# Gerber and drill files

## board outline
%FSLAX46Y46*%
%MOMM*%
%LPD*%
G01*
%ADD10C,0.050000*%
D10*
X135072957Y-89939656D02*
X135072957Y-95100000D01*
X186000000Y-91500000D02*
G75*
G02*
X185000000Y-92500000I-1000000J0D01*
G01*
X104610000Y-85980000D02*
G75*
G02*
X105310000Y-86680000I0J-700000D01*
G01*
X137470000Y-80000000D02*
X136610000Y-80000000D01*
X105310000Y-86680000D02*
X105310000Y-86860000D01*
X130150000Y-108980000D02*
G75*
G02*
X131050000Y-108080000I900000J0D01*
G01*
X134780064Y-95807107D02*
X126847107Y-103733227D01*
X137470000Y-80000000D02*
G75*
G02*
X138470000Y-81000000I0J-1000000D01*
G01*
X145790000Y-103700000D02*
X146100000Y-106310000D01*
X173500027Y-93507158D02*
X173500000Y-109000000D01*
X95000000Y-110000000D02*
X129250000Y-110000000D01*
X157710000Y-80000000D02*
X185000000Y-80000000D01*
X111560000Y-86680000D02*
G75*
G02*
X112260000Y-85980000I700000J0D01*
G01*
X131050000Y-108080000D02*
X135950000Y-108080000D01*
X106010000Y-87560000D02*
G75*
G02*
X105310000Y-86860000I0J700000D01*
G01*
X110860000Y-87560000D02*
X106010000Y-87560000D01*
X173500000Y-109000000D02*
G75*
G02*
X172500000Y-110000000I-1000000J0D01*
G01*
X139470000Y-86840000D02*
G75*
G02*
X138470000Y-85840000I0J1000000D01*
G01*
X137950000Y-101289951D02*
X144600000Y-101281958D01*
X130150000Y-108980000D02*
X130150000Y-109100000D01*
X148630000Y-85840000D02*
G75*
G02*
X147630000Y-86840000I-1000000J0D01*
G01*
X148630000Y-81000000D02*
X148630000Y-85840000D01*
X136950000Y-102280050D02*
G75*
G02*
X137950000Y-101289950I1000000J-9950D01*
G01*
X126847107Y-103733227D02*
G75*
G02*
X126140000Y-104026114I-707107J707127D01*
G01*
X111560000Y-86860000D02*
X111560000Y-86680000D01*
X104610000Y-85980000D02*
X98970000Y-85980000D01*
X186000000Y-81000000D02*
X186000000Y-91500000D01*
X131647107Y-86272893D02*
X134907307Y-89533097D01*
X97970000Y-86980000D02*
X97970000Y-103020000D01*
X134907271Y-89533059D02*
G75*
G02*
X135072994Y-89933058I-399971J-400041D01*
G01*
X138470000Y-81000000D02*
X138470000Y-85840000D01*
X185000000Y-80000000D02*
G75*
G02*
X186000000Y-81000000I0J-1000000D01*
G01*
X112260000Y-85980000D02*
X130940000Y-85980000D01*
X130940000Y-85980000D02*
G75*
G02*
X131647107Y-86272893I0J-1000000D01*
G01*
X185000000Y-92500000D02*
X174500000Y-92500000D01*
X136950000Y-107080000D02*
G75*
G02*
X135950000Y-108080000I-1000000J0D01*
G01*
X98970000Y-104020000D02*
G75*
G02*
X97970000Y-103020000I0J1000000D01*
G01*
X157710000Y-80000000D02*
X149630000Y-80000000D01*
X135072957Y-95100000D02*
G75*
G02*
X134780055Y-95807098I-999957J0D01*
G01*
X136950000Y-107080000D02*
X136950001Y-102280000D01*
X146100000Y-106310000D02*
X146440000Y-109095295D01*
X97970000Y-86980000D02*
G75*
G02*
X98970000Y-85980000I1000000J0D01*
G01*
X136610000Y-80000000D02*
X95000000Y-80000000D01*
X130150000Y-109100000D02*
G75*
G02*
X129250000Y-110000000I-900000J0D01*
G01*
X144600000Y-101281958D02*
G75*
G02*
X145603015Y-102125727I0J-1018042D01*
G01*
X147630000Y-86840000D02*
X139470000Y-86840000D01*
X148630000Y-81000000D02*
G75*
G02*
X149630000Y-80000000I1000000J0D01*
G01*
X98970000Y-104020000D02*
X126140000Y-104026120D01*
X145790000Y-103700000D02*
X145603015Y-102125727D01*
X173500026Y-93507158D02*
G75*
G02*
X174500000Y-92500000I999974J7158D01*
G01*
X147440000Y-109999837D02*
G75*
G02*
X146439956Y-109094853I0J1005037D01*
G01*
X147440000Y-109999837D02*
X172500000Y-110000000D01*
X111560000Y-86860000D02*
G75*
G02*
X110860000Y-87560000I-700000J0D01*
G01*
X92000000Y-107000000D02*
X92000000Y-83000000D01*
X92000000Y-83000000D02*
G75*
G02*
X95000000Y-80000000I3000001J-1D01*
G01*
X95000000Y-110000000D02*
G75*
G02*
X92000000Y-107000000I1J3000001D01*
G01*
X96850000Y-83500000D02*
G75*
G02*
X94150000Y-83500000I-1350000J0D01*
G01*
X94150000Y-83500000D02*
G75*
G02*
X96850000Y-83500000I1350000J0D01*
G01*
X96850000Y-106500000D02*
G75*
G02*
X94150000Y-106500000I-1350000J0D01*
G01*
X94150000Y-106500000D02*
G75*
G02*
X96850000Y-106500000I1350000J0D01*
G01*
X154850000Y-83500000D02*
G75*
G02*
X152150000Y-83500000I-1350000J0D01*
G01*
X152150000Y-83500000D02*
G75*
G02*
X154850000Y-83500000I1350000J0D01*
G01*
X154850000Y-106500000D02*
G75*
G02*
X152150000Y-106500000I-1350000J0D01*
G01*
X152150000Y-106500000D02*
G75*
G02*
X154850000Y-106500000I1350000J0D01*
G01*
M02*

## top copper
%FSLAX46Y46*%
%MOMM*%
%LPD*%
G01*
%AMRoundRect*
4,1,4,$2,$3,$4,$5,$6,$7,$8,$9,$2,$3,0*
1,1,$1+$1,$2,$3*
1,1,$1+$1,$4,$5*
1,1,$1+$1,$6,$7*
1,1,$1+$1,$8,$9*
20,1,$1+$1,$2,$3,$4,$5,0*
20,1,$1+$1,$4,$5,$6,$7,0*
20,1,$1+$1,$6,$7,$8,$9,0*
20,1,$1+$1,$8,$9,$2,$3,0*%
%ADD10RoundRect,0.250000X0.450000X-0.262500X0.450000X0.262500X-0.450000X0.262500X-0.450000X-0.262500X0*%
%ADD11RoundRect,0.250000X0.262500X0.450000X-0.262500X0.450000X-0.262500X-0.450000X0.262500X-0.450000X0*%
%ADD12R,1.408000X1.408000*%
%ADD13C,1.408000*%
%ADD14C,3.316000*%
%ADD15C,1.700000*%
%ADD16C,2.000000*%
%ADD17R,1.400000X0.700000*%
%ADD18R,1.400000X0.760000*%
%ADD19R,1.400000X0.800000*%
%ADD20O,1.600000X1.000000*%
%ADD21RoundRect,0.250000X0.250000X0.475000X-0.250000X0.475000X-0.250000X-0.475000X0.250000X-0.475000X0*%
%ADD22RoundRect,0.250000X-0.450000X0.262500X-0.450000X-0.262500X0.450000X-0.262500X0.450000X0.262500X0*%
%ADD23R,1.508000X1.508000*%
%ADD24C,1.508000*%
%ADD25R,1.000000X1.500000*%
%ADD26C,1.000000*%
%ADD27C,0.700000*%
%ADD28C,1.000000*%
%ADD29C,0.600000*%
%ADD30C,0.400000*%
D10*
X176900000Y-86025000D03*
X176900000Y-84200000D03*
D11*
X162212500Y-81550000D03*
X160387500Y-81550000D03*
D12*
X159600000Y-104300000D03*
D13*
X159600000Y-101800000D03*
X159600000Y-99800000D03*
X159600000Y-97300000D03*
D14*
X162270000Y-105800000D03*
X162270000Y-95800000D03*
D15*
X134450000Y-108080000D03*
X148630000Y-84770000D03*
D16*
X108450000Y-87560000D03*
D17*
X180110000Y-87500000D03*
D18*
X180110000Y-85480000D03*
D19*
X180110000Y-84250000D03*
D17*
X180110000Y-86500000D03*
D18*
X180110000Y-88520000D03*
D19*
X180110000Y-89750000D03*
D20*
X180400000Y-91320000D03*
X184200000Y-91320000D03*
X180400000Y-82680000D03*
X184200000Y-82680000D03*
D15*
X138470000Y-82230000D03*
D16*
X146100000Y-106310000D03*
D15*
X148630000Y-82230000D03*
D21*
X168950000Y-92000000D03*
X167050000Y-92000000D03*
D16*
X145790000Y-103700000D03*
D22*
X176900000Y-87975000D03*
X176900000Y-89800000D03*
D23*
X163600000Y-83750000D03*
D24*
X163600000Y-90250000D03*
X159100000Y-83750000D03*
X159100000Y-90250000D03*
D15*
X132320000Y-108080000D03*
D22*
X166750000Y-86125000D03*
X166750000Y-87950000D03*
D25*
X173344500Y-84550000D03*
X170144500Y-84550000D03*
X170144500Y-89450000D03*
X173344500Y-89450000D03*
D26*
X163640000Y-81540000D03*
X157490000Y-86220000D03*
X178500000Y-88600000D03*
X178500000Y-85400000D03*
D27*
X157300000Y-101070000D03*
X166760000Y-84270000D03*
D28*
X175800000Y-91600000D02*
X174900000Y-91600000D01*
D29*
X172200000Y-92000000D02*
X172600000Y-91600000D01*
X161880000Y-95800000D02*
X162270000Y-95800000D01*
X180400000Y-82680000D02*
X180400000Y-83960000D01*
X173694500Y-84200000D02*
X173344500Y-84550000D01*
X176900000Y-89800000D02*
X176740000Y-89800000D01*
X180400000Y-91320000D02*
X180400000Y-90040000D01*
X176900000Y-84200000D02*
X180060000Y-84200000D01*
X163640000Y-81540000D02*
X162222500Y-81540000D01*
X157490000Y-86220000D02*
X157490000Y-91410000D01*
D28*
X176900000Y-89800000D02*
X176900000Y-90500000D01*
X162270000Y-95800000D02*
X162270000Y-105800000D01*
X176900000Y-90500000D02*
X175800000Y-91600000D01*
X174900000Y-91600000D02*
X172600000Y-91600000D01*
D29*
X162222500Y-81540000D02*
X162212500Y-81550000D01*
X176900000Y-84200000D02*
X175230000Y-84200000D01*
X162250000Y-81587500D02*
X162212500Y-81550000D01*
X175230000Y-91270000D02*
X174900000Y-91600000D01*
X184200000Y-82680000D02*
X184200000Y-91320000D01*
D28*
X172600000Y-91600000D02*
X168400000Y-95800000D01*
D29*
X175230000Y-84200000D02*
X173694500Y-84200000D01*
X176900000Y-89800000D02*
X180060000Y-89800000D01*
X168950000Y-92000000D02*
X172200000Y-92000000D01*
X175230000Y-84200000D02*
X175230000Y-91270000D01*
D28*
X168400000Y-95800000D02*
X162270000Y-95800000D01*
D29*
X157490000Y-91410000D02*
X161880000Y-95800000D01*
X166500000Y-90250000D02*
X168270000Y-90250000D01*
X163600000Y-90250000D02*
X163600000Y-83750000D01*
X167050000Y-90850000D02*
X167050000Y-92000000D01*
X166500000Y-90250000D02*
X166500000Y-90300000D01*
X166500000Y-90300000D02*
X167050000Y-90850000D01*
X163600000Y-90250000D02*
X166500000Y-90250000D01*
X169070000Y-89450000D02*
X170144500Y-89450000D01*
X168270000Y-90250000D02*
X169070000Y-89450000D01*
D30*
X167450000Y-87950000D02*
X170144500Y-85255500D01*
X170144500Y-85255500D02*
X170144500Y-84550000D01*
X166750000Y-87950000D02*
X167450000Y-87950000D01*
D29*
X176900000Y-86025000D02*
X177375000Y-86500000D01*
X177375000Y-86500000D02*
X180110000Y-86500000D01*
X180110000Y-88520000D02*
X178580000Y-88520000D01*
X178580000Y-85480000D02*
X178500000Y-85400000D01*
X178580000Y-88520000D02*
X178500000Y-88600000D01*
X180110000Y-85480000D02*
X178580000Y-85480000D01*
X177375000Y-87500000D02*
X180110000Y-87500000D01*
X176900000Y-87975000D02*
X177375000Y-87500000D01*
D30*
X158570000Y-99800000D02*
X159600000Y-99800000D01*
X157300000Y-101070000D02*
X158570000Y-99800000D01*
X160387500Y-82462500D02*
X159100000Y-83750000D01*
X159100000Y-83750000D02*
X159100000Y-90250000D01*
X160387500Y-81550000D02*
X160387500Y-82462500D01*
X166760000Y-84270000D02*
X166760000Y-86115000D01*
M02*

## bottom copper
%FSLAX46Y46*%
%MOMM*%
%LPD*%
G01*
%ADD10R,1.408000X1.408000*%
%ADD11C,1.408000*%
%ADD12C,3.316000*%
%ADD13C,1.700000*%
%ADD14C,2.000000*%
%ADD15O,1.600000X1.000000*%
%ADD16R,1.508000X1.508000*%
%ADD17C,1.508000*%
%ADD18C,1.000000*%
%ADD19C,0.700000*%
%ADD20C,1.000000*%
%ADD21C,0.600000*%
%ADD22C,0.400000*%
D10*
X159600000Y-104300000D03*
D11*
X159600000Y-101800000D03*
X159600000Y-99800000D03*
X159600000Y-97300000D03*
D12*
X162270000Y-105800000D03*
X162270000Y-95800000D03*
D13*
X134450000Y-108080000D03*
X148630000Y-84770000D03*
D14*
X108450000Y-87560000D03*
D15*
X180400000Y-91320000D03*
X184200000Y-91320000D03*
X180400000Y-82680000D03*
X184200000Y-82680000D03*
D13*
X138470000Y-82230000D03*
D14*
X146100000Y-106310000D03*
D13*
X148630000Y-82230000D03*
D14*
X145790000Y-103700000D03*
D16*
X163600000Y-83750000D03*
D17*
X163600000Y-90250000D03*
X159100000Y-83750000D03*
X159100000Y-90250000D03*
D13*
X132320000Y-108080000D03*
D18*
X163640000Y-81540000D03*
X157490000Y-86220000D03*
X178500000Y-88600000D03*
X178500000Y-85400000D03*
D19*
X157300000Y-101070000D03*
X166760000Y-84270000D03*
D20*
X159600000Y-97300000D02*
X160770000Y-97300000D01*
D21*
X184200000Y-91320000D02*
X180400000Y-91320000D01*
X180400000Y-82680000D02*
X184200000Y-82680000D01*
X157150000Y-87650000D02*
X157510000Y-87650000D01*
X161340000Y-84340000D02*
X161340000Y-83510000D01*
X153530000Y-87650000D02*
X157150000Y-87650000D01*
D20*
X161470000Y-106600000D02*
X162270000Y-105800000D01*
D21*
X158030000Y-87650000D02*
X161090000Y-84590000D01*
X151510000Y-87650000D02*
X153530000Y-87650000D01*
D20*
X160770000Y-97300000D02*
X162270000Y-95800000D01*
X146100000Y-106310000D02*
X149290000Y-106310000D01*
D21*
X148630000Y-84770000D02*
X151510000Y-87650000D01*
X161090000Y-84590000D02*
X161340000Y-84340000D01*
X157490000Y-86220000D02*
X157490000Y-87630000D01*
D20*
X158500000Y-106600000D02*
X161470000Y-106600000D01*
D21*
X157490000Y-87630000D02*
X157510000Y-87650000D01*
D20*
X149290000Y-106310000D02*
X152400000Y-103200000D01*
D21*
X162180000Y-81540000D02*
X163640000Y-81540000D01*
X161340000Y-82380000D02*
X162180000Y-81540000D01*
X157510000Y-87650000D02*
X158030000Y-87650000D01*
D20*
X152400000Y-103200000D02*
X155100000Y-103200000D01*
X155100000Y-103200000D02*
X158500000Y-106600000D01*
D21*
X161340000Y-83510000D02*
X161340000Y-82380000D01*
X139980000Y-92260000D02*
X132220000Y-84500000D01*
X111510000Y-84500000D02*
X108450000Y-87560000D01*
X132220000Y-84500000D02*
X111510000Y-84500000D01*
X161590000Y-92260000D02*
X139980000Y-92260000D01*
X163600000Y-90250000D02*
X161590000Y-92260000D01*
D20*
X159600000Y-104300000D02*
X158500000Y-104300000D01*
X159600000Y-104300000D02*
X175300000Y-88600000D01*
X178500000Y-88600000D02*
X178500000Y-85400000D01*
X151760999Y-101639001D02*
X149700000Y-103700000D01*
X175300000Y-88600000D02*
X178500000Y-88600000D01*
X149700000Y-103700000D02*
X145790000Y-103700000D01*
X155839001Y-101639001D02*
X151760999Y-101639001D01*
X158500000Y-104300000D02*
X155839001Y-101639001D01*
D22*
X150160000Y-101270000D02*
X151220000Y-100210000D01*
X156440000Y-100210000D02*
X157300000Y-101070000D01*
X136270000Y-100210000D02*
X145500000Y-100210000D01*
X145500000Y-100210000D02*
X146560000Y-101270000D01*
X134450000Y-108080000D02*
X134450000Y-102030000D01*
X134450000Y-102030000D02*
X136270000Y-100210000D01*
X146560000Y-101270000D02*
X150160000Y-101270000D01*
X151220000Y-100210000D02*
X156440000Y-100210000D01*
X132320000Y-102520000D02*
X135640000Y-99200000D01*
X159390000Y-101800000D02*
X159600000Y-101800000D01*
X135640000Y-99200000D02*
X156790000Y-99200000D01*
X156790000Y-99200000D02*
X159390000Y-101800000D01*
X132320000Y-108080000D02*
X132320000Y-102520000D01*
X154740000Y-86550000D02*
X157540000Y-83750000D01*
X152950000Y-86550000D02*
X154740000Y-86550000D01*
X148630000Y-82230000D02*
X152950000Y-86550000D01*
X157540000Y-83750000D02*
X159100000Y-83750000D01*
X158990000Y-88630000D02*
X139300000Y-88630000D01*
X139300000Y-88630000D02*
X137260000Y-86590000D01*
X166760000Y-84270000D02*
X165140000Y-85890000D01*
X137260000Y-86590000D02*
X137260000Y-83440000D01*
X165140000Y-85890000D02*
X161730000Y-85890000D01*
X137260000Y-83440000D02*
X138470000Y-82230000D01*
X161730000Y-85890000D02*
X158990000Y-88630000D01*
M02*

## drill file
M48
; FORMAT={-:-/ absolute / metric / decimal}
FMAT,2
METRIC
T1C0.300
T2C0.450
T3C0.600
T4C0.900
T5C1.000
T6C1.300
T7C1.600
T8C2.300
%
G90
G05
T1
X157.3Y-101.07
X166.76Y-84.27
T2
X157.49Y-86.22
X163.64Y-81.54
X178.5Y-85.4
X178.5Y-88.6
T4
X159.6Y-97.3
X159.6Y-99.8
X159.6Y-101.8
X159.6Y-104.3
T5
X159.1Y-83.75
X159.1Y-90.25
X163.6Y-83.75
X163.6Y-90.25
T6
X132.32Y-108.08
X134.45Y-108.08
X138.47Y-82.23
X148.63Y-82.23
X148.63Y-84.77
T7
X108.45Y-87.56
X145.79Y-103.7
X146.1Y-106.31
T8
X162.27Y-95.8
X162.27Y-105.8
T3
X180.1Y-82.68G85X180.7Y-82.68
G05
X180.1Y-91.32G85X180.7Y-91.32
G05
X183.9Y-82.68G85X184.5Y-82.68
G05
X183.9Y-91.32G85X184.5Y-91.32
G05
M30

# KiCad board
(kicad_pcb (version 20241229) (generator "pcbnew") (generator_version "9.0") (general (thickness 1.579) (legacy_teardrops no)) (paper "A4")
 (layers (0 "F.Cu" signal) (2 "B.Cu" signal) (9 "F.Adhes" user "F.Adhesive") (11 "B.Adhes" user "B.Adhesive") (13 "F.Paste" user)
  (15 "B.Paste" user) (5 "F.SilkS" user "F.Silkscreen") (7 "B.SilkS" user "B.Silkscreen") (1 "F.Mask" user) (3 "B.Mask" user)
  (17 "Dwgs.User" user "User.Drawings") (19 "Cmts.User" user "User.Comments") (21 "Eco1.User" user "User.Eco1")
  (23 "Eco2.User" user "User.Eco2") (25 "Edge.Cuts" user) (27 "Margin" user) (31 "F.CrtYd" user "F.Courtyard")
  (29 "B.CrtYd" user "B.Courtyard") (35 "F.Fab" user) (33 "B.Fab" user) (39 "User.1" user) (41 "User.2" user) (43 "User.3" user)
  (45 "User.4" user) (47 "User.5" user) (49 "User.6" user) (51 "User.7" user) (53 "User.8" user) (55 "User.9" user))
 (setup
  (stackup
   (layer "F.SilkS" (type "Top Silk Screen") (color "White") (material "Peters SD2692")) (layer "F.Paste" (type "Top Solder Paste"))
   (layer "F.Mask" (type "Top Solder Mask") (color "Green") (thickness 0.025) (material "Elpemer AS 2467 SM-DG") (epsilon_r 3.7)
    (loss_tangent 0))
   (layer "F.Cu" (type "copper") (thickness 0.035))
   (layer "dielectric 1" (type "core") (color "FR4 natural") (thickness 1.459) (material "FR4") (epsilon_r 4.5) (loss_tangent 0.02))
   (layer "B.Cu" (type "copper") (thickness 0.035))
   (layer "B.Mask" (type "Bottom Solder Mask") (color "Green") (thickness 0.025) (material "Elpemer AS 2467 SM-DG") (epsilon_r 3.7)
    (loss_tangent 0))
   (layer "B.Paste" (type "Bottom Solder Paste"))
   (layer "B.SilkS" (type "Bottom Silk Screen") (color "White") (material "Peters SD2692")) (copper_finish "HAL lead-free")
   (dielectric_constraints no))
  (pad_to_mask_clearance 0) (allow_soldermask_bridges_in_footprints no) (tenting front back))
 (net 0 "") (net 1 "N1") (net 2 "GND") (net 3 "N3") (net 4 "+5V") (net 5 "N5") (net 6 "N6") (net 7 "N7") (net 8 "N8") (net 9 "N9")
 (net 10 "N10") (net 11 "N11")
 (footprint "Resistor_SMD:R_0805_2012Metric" (layer "F.Cu") (at 176.9 85.1125 90)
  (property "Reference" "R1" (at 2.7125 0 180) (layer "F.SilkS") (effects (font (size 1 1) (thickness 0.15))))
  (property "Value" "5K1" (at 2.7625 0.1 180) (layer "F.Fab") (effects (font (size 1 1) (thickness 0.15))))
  (pad "1" smd roundrect (at -0.9125 0 90) (size 1.025 1.4) (layers "F.Cu" "F.Mask" "F.Paste") (roundrect_rratio 0.243902) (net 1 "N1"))
  (pad "2" smd roundrect (at 0.9125 0 90) (size 1.025 1.4) (layers "F.Cu" "F.Mask" "F.Paste") (roundrect_rratio 0.243902) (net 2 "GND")))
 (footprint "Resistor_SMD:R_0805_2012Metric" (layer "F.Cu") (at 161.3 81.55 180)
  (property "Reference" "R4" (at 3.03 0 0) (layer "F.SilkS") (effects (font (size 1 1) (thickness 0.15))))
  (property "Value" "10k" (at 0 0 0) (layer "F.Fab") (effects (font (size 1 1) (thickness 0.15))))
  (pad "1" smd roundrect (at -0.9125 0 180) (size 1.025 1.4) (layers "F.Cu" "F.Mask" "F.Paste") (roundrect_rratio 0.243902) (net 2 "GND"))
  (pad "2" smd roundrect (at 0.9125 0 180) (size 1.025 1.4) (layers "F.Cu" "F.Mask" "F.Paste") (roundrect_rratio 0.243902) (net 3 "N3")))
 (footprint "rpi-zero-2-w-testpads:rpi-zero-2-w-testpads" (layer "F.Cu") (at 157 110)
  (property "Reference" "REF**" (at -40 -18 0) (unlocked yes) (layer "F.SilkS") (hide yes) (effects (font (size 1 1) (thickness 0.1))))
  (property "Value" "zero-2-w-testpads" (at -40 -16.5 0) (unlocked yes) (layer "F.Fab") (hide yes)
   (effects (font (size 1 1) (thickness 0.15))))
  (fp_line (start -65 -3) (end -65 -27) (stroke (width 0.05) (type solid)) (layer "Edge.Cuts"))
  (fp_arc (start -65 -27) (mid -64.12132 -29.12132) (end -62 -30) (stroke (width 0.05) (type solid)) (layer "Edge.Cuts"))
  (fp_arc (start -62 0) (mid -64.12132 -0.87868) (end -65 -3) (stroke (width 0.05) (type solid)) (layer "Edge.Cuts"))
  (fp_circle (center -61.5 -26.5) (end -60.15 -26.5) (stroke (width 0.05) (type solid)) (fill no) (layer "Edge.Cuts"))
  (fp_circle (center -61.5 -3.5) (end -60.15 -3.5) (stroke (width 0.05) (type solid)) (fill no) (layer "Edge.Cuts"))
  (fp_circle (center -3.5 -26.5) (end -2.15 -26.5) (stroke (width 0.05) (type solid)) (fill no) (layer "Edge.Cuts"))
  (fp_circle (center -3.5 -3.5) (end -2.15 -3.5) (stroke (width 0.05) (type solid)) (fill no) (layer "Edge.Cuts"))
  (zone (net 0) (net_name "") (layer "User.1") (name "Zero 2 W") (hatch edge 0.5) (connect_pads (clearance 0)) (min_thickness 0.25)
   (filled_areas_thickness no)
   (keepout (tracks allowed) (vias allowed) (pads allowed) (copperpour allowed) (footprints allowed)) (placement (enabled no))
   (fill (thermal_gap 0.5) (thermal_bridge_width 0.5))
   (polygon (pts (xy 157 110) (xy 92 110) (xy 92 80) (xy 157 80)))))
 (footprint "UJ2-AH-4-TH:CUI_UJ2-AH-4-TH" (layer "F.Cu") (at 159.6 104.3 90)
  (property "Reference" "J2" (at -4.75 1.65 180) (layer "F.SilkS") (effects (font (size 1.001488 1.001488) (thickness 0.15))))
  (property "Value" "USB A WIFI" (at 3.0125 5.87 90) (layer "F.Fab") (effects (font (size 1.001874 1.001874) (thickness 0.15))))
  (pad "1" thru_hole rect (at 0 0 90) (size 1.408 1.408) (drill 0.9) (layers "*.Cu" "*.Mask") (remove_unused_layers no) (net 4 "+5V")
   (solder_mask_margin 0.102))
  (pad "2" thru_hole circle (at 2.5 0 90) (size 1.408 1.408) (drill 0.9) (layers "*.Cu" "*.Mask") (remove_unused_layers no) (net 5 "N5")
   (solder_mask_margin 0.102))
  (pad "3" thru_hole circle (at 4.5 0 90) (size 1.408 1.408) (drill 0.9) (layers "*.Cu" "*.Mask") (remove_unused_layers no) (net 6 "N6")
   (solder_mask_margin 0.102))
  (pad "4" thru_hole circle (at 7 0 90) (size 1.408 1.408) (drill 0.9) (layers "*.Cu" "*.Mask") (remove_unused_layers no) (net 2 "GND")
   (solder_mask_margin 0.102))
  (pad "SH1" thru_hole circle (at -1.5 2.67 90) (size 3.316 3.316) (drill 2.3) (layers "*.Cu" "*.Mask") (remove_unused_layers no)
   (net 2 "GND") (solder_mask_margin 0.102))
  (pad "SH2" thru_hole circle (at 8.5 2.67 90) (size 3.316 3.316) (drill 2.3) (layers "*.Cu" "*.Mask") (remove_unused_layers no)
   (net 2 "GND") (solder_mask_margin 0.102)))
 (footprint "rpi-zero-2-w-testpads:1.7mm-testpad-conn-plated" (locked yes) (layer "F.Cu") (at 134.45 108.08)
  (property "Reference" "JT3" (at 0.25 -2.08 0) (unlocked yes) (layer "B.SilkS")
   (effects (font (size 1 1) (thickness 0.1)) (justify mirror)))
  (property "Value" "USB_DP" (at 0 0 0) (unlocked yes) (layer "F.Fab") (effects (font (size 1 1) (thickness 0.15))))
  (pad "1" thru_hole circle (at 0 0) (size 1.7 1.7) (drill 1.3) (layers "*.Cu" "*.Mask") (remove_unused_layers no) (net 6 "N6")))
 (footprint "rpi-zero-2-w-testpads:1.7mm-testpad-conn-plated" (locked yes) (layer "F.Cu") (at 148.63 84.77)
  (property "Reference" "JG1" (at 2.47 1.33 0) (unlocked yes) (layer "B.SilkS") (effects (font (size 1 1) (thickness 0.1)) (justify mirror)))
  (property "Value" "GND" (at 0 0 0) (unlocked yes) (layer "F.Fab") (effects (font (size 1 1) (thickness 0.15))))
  (pad "1" thru_hole circle (at 0 0) (size 1.7 1.7) (drill 1.3) (layers "*.Cu" "*.Mask") (remove_unused_layers no) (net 2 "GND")))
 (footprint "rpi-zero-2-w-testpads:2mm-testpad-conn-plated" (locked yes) (layer "F.Cu") (at 108.45 87.56)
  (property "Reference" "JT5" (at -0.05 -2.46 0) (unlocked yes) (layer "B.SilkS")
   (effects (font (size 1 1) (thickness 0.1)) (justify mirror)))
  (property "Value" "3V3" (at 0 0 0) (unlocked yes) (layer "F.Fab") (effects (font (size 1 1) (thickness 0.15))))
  (pad "1" thru_hole circle (at 0 0) (size 2 2) (drill 1.6) (layers "*.Cu" "*.Mask") (remove_unused_layers no) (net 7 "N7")))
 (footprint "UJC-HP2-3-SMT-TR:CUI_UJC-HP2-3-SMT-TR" (layer "F.Cu") (at 184.2 87 90)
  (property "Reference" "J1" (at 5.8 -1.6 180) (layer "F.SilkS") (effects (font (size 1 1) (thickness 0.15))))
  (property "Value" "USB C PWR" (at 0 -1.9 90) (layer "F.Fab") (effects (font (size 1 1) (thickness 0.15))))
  (pad "A5" smd rect (at -0.5 -4.09 90) (size 0.7 1.4) (layers "F.Cu" "F.Mask" "F.Paste") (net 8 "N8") (solder_mask_margin 0.102))
  (pad "A9" smd rect (at 1.52 -4.09 90) (size 0.76 1.4) (layers "F.Cu" "F.Mask" "F.Paste") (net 4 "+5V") (solder_mask_margin 0.102))
  (pad "A12" smd rect (at 2.75 -4.09 90) (size 0.8 1.4) (layers "F.Cu" "F.Mask" "F.Paste") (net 2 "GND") (solder_mask_margin 0.102))
  (pad "B5" smd rect (at 0.5 -4.09 90) (size 0.7 1.4) (layers "F.Cu" "F.Mask" "F.Paste") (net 1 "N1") (solder_mask_margin 0.102))
  (pad "B9" smd rect (at -1.52 -4.09 90) (size 0.76 1.4) (layers "F.Cu" "F.Mask" "F.Paste") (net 4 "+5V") (solder_mask_margin 0.102))
  (pad "B12" smd rect (at -2.75 -4.09 90) (size 0.8 1.4) (layers "F.Cu" "F.Mask" "F.Paste") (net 2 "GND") (solder_mask_margin 0.102))
  (pad "SH1" thru_hole oval (at -4.32 -3.8 90) (size 1 1.6) (drill oval 0.6 1.2) (layers "*.Cu" "*.Mask") (remove_unused_layers no)
   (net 2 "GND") (solder_mask_margin 0.102))
  (pad "SH2" thru_hole oval (at -4.32 0 90) (size 1 1.6) (drill oval 0.6 1.2) (layers "*.Cu" "*.Mask") (remove_unused_layers no)
   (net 2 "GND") (solder_mask_margin 0.102))
  (pad "SH3" thru_hole oval (at 4.32 -3.8 90) (size 1 1.6) (drill oval 0.6 1.2) (layers "*.Cu" "*.Mask") (remove_unused_layers no)
   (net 2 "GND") (solder_mask_margin 0.102))
  (pad "SH4" thru_hole oval (at 4.32 0 90) (size 1 1.6) (drill oval 0.6 1.2) (layers "*.Cu" "*.Mask") (remove_unused_layers no)
   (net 2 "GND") (solder_mask_margin 0.102)))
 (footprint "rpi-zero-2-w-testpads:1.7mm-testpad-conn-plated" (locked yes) (layer "F.Cu") (at 138.47 82.23)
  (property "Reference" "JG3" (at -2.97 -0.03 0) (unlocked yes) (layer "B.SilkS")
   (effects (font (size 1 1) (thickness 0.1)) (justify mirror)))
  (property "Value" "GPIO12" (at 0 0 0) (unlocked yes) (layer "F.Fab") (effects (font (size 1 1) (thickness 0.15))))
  (pad "1" thru_hole circle (at 0 0) (size 1.7 1.7) (drill 1.3) (layers "*.Cu" "*.Mask") (remove_unused_layers no) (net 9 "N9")))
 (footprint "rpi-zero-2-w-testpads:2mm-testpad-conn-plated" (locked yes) (layer "F.Cu") (at 146.1 106.31)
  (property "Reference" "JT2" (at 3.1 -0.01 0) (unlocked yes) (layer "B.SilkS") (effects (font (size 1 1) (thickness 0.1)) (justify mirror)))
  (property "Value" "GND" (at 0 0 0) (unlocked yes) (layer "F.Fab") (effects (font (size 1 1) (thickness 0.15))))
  (pad "1" thru_hole circle (at 0 0) (size 2 2) (drill 1.6) (layers "*.Cu" "*.Mask") (remove_unused_layers no) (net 2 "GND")))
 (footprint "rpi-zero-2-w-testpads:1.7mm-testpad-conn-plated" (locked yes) (layer "F.Cu") (at 148.63 82.23)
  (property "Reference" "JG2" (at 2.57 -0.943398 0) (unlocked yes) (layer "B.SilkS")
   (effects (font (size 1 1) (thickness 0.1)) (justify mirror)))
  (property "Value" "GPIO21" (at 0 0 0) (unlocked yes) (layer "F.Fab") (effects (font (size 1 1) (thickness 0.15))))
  (pad "1" thru_hole circle (at 0 0) (size 1.7 1.7) (drill 1.3) (layers "*.Cu" "*.Mask") (remove_unused_layers no) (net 3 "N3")))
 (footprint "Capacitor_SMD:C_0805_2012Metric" (layer "F.Cu") (at 168 92 180)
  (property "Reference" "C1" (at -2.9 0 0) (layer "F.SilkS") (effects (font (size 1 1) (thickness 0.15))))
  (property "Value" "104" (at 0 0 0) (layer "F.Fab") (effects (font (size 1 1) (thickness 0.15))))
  (pad "1" smd roundrect (at -0.95 0 180) (size 1 1.45) (layers "F.Cu" "F.Mask" "F.Paste") (roundrect_rratio 0.25) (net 2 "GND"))
  (pad "2" smd roundrect (at 0.95 0 180) (size 1 1.45) (layers "F.Cu" "F.Mask" "F.Paste") (roundrect_rratio 0.25) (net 7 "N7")))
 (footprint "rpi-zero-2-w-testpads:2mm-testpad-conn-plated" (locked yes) (layer "F.Cu") (at 145.79 103.7)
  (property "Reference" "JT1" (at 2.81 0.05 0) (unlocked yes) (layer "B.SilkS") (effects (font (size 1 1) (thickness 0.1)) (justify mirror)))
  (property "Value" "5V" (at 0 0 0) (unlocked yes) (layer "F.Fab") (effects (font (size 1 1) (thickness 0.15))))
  (pad "1" thru_hole circle (at 0 0) (size 2 2) (drill 1.6) (layers "*.Cu" "*.Mask") (remove_unused_layers no) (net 4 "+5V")))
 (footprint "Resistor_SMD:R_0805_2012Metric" (layer "F.Cu") (at 176.9 88.8875 -90)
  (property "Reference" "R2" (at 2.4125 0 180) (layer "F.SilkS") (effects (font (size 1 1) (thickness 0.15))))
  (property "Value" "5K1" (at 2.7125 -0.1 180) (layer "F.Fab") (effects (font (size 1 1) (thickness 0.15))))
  (pad "1" smd roundrect (at -0.9125 0 270) (size 1.025 1.4) (layers "F.Cu" "F.Mask" "F.Paste") (roundrect_rratio 0.243902) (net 8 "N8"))
  (pad "2" smd roundrect (at 0.9125 0 270) (size 1.025 1.4) (layers "F.Cu" "F.Mask" "F.Paste") (roundrect_rratio 0.243902) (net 2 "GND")))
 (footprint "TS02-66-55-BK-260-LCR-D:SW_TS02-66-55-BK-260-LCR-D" (layer "F.Cu") (at 161.35 87 -90)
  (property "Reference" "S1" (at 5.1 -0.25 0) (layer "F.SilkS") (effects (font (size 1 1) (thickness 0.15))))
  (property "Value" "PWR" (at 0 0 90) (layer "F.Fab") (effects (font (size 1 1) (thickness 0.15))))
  (pad "1" thru_hole rect (at -3.25 -2.25 270) (size 1.508 1.508) (drill 1) (layers "*.Cu" "*.Mask") (remove_unused_layers no) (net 7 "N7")
   (solder_mask_margin 0.102))
  (pad "2" thru_hole circle (at 3.25 -2.25 270) (size 1.508 1.508) (drill 1) (layers "*.Cu" "*.Mask") (remove_unused_layers no) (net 7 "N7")
   (solder_mask_margin 0.102))
  (pad "3" thru_hole circle (at -3.25 2.25 270) (size 1.508 1.508) (drill 1) (layers "*.Cu" "*.Mask") (remove_unused_layers no) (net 3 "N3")
   (solder_mask_margin 0.102))
  (pad "4" thru_hole circle (at 3.25 2.25 270) (size 1.508 1.508) (drill 1) (layers "*.Cu" "*.Mask") (remove_unused_layers no) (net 3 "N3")
   (solder_mask_margin 0.102)))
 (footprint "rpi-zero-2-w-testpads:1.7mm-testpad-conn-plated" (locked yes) (layer "F.Cu") (at 132.32 108.08)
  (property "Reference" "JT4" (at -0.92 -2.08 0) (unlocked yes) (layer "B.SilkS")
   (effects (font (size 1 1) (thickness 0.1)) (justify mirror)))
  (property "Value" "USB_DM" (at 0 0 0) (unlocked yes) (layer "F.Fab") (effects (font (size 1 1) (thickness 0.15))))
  (pad "1" thru_hole circle (at 0 0) (size 1.7 1.7) (drill 1.3) (layers "*.Cu" "*.Mask") (remove_unused_layers no) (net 5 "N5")))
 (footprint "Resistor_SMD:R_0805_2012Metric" (layer "F.Cu") (at 166.75 87.0375 -90)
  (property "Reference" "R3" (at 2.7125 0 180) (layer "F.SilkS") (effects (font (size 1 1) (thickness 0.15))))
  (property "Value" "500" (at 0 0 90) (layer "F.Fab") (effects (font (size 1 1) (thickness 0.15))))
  (pad "1" smd roundrect (at -0.9125 0 270) (size 1.025 1.4) (layers "F.Cu" "F.Mask" "F.Paste") (roundrect_rratio 0.243902) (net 9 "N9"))
  (pad "2" smd roundrect (at 0.9125 0 270) (size 1.025 1.4) (layers "F.Cu" "F.Mask" "F.Paste") (roundrect_rratio 0.243902) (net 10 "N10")))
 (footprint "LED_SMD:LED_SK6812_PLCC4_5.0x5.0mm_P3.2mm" (layer "F.Cu") (at 171.7445 87 -90)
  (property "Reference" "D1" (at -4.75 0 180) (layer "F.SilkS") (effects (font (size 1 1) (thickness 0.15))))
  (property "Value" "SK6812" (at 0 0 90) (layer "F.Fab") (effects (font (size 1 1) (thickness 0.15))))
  (pad "1" smd rect (at -2.45 -1.6 90) (size 1.5 1) (layers "F.Cu" "F.Mask" "F.Paste") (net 2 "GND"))
  (pad "2" smd rect (at -2.45 1.6 90) (size 1.5 1) (layers "F.Cu" "F.Mask" "F.Paste") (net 10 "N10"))
  (pad "3" smd rect (at 2.45 1.6 90) (size 1.5 1) (layers "F.Cu" "F.Mask" "F.Paste") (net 7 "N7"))
  (pad "4" smd rect (at 2.45 -1.6 90) (size 1.5 1) (layers "F.Cu" "F.Mask" "F.Paste") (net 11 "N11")))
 (gr_line (start 135.072957 89.939656) (end 135.072957 95.1) (stroke (width 0.05) (type default)) (layer "Edge.Cuts"))
 (gr_arc (start 186 91.5) (mid 185.707107 92.207107) (end 185 92.5) (stroke (width 0.05) (type default)) (layer "Edge.Cuts"))
 (gr_arc (start 104.61 85.98) (mid 105.104975 86.185025) (end 105.31 86.68) (stroke (width 0.05) (type default)) (layer "Edge.Cuts"))
 (gr_line (start 137.47 80) (end 136.61 80) (stroke (width 0.05) (type default)) (layer "Edge.Cuts"))
 (gr_line (start 105.31 86.68) (end 105.31 86.86) (stroke (width 0.05) (type default)) (layer "Edge.Cuts"))
 (gr_arc (start 130.15 108.98) (mid 130.413604 108.343604) (end 131.05 108.08) (stroke (width 0.05) (type default)) (layer "Edge.Cuts"))
 (gr_line (start 134.780064 95.807107) (end 126.847107 103.733227) (stroke (width 0.05) (type solid)) (layer "Edge.Cuts"))
 (gr_arc (start 137.47 80) (mid 138.177107 80.292893) (end 138.47 81) (stroke (width 0.05) (type default)) (layer "Edge.Cuts"))
 (gr_line (start 145.79 103.7) (end 146.1 106.31) (stroke (width 0.05) (type solid)) (layer "Edge.Cuts"))
 (gr_line (start 173.500027 93.507158) (end 173.5 109) (stroke (width 0.05) (type default)) (layer "Edge.Cuts"))
 (gr_line (start 95 110) (end 129.25 110) (stroke (width 0.05) (type default)) (layer "Edge.Cuts"))
 (gr_line (start 157.71 80) (end 185 80) (stroke (width 0.05) (type solid)) (layer "Edge.Cuts"))
 (gr_arc (start 111.56 86.68) (mid 111.765025 86.185025) (end 112.26 85.98) (stroke (width 0.05) (type default)) (layer "Edge.Cuts"))
 (gr_line (start 131.05 108.08) (end 135.95 108.08) (stroke (width 0.05) (type solid)) (layer "Edge.Cuts"))
 (gr_arc (start 106.01 87.56) (mid 105.515025 87.354975) (end 105.31 86.86) (stroke (width 0.05) (type default)) (layer "Edge.Cuts"))
 (gr_line (start 110.86 87.56) (end 106.01 87.56) (stroke (width 0.05) (type solid)) (layer "Edge.Cuts"))
 (gr_arc (start 173.5 109) (mid 173.207107 109.707107) (end 172.5 110) (stroke (width 0.05) (type default)) (layer "Edge.Cuts"))
 (gr_arc (start 139.47 86.84) (mid 138.762893 86.547107) (end 138.47 85.84) (stroke (width 0.05) (type default)) (layer "Edge.Cuts"))
 (gr_line (start 137.95 101.289951) (end 144.6 101.281958) (stroke (width 0.05) (type default)) (layer "Edge.Cuts"))
 (gr_line (start 130.15 108.98) (end 130.15 109.1) (stroke (width 0.05) (type default)) (layer "Edge.Cuts"))
 (gr_arc (start 148.63 85.84) (mid 148.337107 86.547107) (end 147.63 86.84) (stroke (width 0.05) (type default)) (layer "Edge.Cuts"))
 (gr_line (start 148.63 81) (end 148.63 85.84) (stroke (width 0.05) (type solid)) (layer "Edge.Cuts"))
 (gr_arc (start 136.95 102.28005) (mid 137.246402 101.579381) (end 137.95 101.29) (stroke (width 0.05) (type default)) (layer "Edge.Cuts"))
 (gr_arc (start 126.847107 103.733227) (mid 126.522684 103.95) (end 126.14 104.02612) (stroke (width 0.05) (type default))
  (layer "Edge.Cuts"))
 (gr_line (start 111.56 86.86) (end 111.56 86.68) (stroke (width 0.05) (type default)) (layer "Edge.Cuts"))
 (gr_line (start 104.61 85.98) (end 98.97 85.98) (stroke (width 0.05) (type default)) (layer "Edge.Cuts"))
 (gr_line (start 186 81) (end 186 91.5) (stroke (width 0.05) (type default)) (layer "Edge.Cuts"))
 (gr_line (start 131.647107 86.272893) (end 134.907307 89.533097) (stroke (width 0.05) (type solid)) (layer "Edge.Cuts"))
 (gr_line (start 97.97 86.98) (end 97.97 103.02) (stroke (width 0.05) (type default)) (layer "Edge.Cuts"))
 (gr_arc (start 134.907271 89.533059) (mid 135.029916 89.716576) (end 135.072994 89.933058) (stroke (width 0.05) (type default))
  (layer "Edge.Cuts"))
 (gr_line (start 138.47 81) (end 138.47 85.84) (stroke (width 0.05) (type solid)) (layer "Edge.Cuts"))
 (gr_arc (start 185 80) (mid 185.707107 80.292893) (end 186 81) (stroke (width 0.05) (type solid)) (layer "Edge.Cuts"))
 (gr_line (start 112.26 85.98) (end 130.94 85.98) (stroke (width 0.05) (type default)) (layer "Edge.Cuts"))
 (gr_arc (start 130.94 85.98) (mid 131.322683 86.05612) (end 131.647107 86.272893) (stroke (width 0.05) (type default)) (layer "Edge.Cuts"))
 (gr_line (start 185 92.5) (end 174.5 92.5) (stroke (width 0.05) (type default)) (layer "Edge.Cuts"))
 (gr_arc (start 136.95 107.08) (mid 136.657107 107.787107) (end 135.95 108.08) (stroke (width 0.05) (type default)) (layer "Edge.Cuts"))
 (gr_arc (start 98.97 104.02) (mid 98.262893 103.727107) (end 97.97 103.02) (stroke (width 0.05) (type default)) (layer "Edge.Cuts"))
 (gr_line (start 157.71 80) (end 149.63 80) (stroke (width 0.05) (type default)) (layer "Edge.Cuts"))
 (gr_arc (start 135.072957 95.1) (mid 134.996837 95.482683) (end 134.780064 95.807107) (stroke (width 0.05) (type default))
  (layer "Edge.Cuts"))
 (gr_line (start 136.95 107.08) (end 136.950001 102.28) (stroke (width 0.05) (type default)) (layer "Edge.Cuts"))
 (gr_line (start 146.1 106.31) (end 146.44 109.095295) (stroke (width 0.05) (type solid)) (layer "Edge.Cuts"))
 (gr_arc (start 97.97 86.98) (mid 98.262893 86.272893) (end 98.97 85.98) (stroke (width 0.05) (type solid)) (layer "Edge.Cuts"))
 (gr_line (start 136.61 80) (end 95 80) (stroke (width 0.05) (type default)) (layer "Edge.Cuts"))
 (gr_arc (start 130.15 109.1) (mid 129.886396 109.736396) (end 129.25 110) (stroke (width 0.05) (type default)) (layer "Edge.Cuts"))
 (gr_arc (start 144.6 101.281958) (mid 145.25536 101.520954) (end 145.603015 102.125727) (stroke (width 0.05) (type default))
  (layer "Edge.Cuts"))
 (gr_line (start 147.63 86.84) (end 139.47 86.84) (stroke (width 0.05) (type default)) (layer "Edge.Cuts"))
 (gr_arc (start 148.63 81) (mid 148.922893 80.292893) (end 149.63 80) (stroke (width 0.05) (type default)) (layer "Edge.Cuts"))
 (gr_line (start 98.97 104.02) (end 126.14 104.02612) (stroke (width 0.05) (type default)) (layer "Edge.Cuts"))
 (gr_line (start 145.79 103.7) (end 145.603015 102.125727) (stroke (width 0.05) (type solid)) (layer "Edge.Cuts"))
 (gr_arc (start 173.500026 93.507158) (mid 173.790367 92.795429) (end 174.5 92.5) (stroke (width 0.05) (type default)) (layer "Edge.Cuts"))
 (gr_arc (start 147.44 109.999837) (mid 146.765648 109.74) (end 146.44 109.094849) (stroke (width 0.05) (type default)) (layer "Edge.Cuts"))
 (gr_line (start 147.44 109.999837) (end 172.5 110) (stroke (width 0.05) (type default)) (layer "Edge.Cuts"))
 (gr_arc (start 111.56 86.86) (mid 111.354975 87.354975) (end 110.86 87.56) (stroke (width 0.05) (type default)) (layer "Edge.Cuts"))
 (segment (start 175.8 91.6) (end 174.9 91.6) (width 1) (layer "F.Cu") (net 2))
 (segment (start 172.2 92) (end 172.6 91.6) (width 0.6) (layer "F.Cu") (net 2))
 (segment (start 161.88 95.8) (end 162.27 95.8) (width 0.6) (layer "F.Cu") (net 2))
 (segment (start 180.4 82.68) (end 180.4 83.96) (width 0.6) (layer "F.Cu") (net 2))
 (segment (start 173.6945 84.2) (end 173.3445 84.55) (width 0.6) (layer "F.Cu") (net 2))
 (segment (start 176.9 89.8) (end 176.74 89.8) (width 0.6) (layer "F.Cu") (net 2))
 (segment (start 180.4 91.32) (end 180.4 90.04) (width 0.6) (layer "F.Cu") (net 2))
 (segment (start 176.9 84.2) (end 180.06 84.2) (width 0.6) (layer "F.Cu") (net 2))
 (segment (start 163.64 81.54) (end 162.2225 81.54) (width 0.6) (layer "F.Cu") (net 2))
 (segment (start 157.49 86.22) (end 157.49 91.41) (width 0.6) (layer "F.Cu") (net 2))
 (segment (start 176.9 89.8) (end 176.9 90.5) (width 1) (layer "F.Cu") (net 2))
 (segment (start 162.27 95.8) (end 162.27 105.8) (width 1) (layer "F.Cu") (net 2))
 (segment (start 176.9 90.5) (end 175.8 91.6) (width 1) (layer "F.Cu") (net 2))
 (segment (start 174.9 91.6) (end 172.6 91.6) (width 1) (layer "F.Cu") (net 2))
 (segment (start 162.2225 81.54) (end 162.2125 81.55) (width 0.6) (layer "F.Cu") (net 2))
 (segment (start 176.9 84.2) (end 175.23 84.2) (width 0.6) (layer "F.Cu") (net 2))
 (segment (start 162.25 81.5875) (end 162.2125 81.55) (width 0.6) (layer "F.Cu") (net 2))
 (segment (start 175.23 91.27) (end 174.9 91.6) (width 0.6) (layer "F.Cu") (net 2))
 (segment (start 184.2 82.68) (end 184.2 91.32) (width 0.6) (layer "F.Cu") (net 2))
 (segment (start 172.6 91.6) (end 168.4 95.8) (width 1) (layer "F.Cu") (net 2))
 (segment (start 175.23 84.2) (end 173.6945 84.2) (width 0.6) (layer "F.Cu") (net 2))
 (segment (start 176.9 89.8) (end 180.06 89.8) (width 0.6) (layer "F.Cu") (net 2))
 (segment (start 168.95 92) (end 172.2 92) (width 0.6) (layer "F.Cu") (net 2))
 (segment (start 175.23 84.2) (end 175.23 91.27) (width 0.6) (layer "F.Cu") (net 2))
 (segment (start 168.4 95.8) (end 162.27 95.8) (width 1) (layer "F.Cu") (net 2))
 (segment (start 157.49 91.41) (end 161.88 95.8) (width 0.6) (layer "F.Cu") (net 2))
 (via (at 163.64 81.54) (size 1) (drill 0.45) (layers "F.Cu" "B.Cu") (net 2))
 (via (at 157.49 86.22) (size 1) (drill 0.45) (layers "F.Cu" "B.Cu") (free yes) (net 2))
 (segment (start 159.6 97.3) (end 160.77 97.3) (width 1) (layer "B.Cu") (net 2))
 (segment (start 184.2 91.32) (end 180.4 91.32) (width 0.6) (layer "B.Cu") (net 2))
 (segment (start 180.4 82.68) (end 184.2 82.68) (width 0.6) (layer "B.Cu") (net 2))
 (segment (start 157.15 87.65) (end 157.51 87.65) (width 0.6) (layer "B.Cu") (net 2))
 (segment (start 161.34 84.34) (end 161.34 83.51) (width 0.6) (layer "B.Cu") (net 2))
 (segment (start 153.53 87.65) (end 157.15 87.65) (width 0.6) (layer "B.Cu") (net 2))
 (segment (start 161.47 106.6) (end 162.27 105.8) (width 1) (layer "B.Cu") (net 2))
 (segment (start 158.03 87.65) (end 161.09 84.59) (width 0.6) (layer "B.Cu") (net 2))
 (segment (start 151.51 87.65) (end 153.53 87.65) (width 0.6) (layer "B.Cu") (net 2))
 (segment (start 160.77 97.3) (end 162.27 95.8) (width 1) (layer "B.Cu") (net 2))
 (segment (start 146.1 106.31) (end 149.29 106.31) (width 1) (layer "B.Cu") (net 2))
 (segment (start 148.63 84.77) (end 151.51 87.65) (width 0.6) (layer "B.Cu") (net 2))
 (segment (start 161.09 84.59) (end 161.34 84.34) (width 0.6) (layer "B.Cu") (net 2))
 (segment (start 157.49 86.22) (end 157.49 87.63) (width 0.6) (layer "B.Cu") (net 2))
 (segment (start 158.5 106.6) (end 161.47 106.6) (width 1) (layer "B.Cu") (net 2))
 (segment (start 157.49 87.63) (end 157.51 87.65) (width 0.6) (layer "B.Cu") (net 2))
 (segment (start 149.29 106.31) (end 152.4 103.2) (width 1) (layer "B.Cu") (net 2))
 (segment (start 162.18 81.54) (end 163.64 81.54) (width 0.6) (layer "B.Cu") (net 2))
 (segment (start 161.34 82.38) (end 162.18 81.54) (width 0.6) (layer "B.Cu") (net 2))
 (segment (start 157.51 87.65) (end 158.03 87.65) (width 0.6) (layer "B.Cu") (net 2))
 (segment (start 152.4 103.2) (end 155.1 103.2) (width 1) (layer "B.Cu") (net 2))
 (segment (start 155.1 103.2) (end 158.5 106.6) (width 1) (layer "B.Cu") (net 2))
 (segment (start 161.34 83.51) (end 161.34 82.38) (width 0.6) (layer "B.Cu") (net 2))
 (segment (start 166.5 90.25) (end 168.27 90.25) (width 0.6) (layer "F.Cu") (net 7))
 (segment (start 163.6 90.25) (end 163.6 83.75) (width 0.6) (layer "F.Cu") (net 7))
 (segment (start 167.05 90.85) (end 167.05 92) (width 0.6) (layer "F.Cu") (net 7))
 (segment (start 166.5 90.25) (end 166.5 90.3) (width 0.6) (layer "F.Cu") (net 7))
 (segment (start 166.5 90.3) (end 167.05 90.85) (width 0.6) (layer "F.Cu") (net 7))
 (segment (start 163.6 90.25) (end 166.5 90.25) (width 0.6) (layer "F.Cu") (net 7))
 (segment (start 169.07 89.45) (end 170.1445 89.45) (width 0.6) (layer "F.Cu") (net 7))
 (segment (start 168.27 90.25) (end 169.07 89.45) (width 0.6) (layer "F.Cu") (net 7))
 (segment (start 139.98 92.26) (end 132.22 84.5) (width 0.6) (layer "B.Cu") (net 7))
 (segment (start 111.51 84.5) (end 108.45 87.56) (width 0.6) (layer "B.Cu") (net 7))
 (segment (start 132.22 84.5) (end 111.51 84.5) (width 0.6) (layer "B.Cu") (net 7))
 (segment (start 161.59 92.26) (end 139.98 92.26) (width 0.6) (layer "B.Cu") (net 7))
 (segment (start 163.6 90.25) (end 161.59 92.26) (width 0.6) (layer "B.Cu") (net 7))
 (segment (start 167.45 87.95) (end 170.1445 85.2555) (width 0.4) (layer "F.Cu") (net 10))
 (segment (start 170.1445 85.2555) (end 170.1445 84.55) (width 0.4) (layer "F.Cu") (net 10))
 (segment (start 166.75 87.95) (end 167.45 87.95) (width 0.4) (layer "F.Cu") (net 10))
 (segment (start 176.9 86.025) (end 177.375 86.5) (width 0.6) (layer "F.Cu") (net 1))
 (segment (start 177.375 86.5) (end 180.11 86.5) (width 0.6) (layer "F.Cu") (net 1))
 (segment (start 180.11 88.52) (end 178.58 88.52) (width 0.6) (layer "F.Cu") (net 4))
 (segment (start 178.58 85.48) (end 178.5 85.4) (width 0.6) (layer "F.Cu") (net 4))
 (segment (start 178.58 88.52) (end 178.5 88.6) (width 0.6) (layer "F.Cu") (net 4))
 (segment (start 180.11 85.48) (end 178.58 85.48) (width 0.6) (layer "F.Cu") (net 4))
 (via (at 178.5 88.6) (size 1) (drill 0.45) (layers "F.Cu" "B.Cu") (free yes) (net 4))
 (via (at 178.5 85.4) (size 1) (drill 0.45) (layers "F.Cu" "B.Cu") (free yes) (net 4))
 (segment (start 159.6 104.3) (end 158.5 104.3) (width 1) (layer "B.Cu") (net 4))
 (segment (start 159.6 104.3) (end 175.3 88.6) (width 1) (layer "B.Cu") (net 4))
 (segment (start 178.5 88.6) (end 178.5 85.4) (width 1) (layer "B.Cu") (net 4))
 (segment (start 151.760999 101.639001) (end 149.7 103.7) (width 1) (layer "B.Cu") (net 4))
 (segment (start 175.3 88.6) (end 178.5 88.6) (width 1) (layer "B.Cu") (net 4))
 (segment (start 149.7 103.7) (end 145.79 103.7) (width 1) (layer "B.Cu") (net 4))
 (segment (start 155.839001 101.639001) (end 151.760999 101.639001) (width 1) (layer "B.Cu") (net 4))
 (segment (start 158.5 104.3) (end 155.839001 101.639001) (width 1) (layer "B.Cu") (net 4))
 (segment (start 177.375 87.5) (end 180.11 87.5) (width 0.6) (layer "F.Cu") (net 8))
 (segment (start 176.9 87.975) (end 177.375 87.5) (width 0.6) (layer "F.Cu") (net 8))
 (segment (start 158.57 99.8) (end 159.6 99.8) (width 0.4) (layer "F.Cu") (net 6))
 (segment (start 157.3 101.07) (end 158.57 99.8) (width 0.4) (layer "F.Cu") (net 6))
 (via (at 157.3 101.07) (size 0.7) (drill 0.3) (layers "F.Cu" "B.Cu") (free yes) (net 6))
 (segment (start 150.16 101.27) (end 151.22 100.21) (width 0.4) (layer "B.Cu") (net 6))
 (segment (start 156.44 100.21) (end 157.3 101.07) (width 0.4) (layer "B.Cu") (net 6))
 (segment (start 136.27 100.21) (end 145.5 100.21) (width 0.4) (layer "B.Cu") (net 6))
 (segment (start 145.5 100.21) (end 146.56 101.27) (width 0.4) (layer "B.Cu") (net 6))
 (segment (start 134.45 108.08) (end 134.45 102.03) (width 0.4) (layer "B.Cu") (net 6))
 (segment (start 134.45 102.03) (end 136.27 100.21) (width 0.4) (layer "B.Cu") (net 6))
 (segment (start 146.56 101.27) (end 150.16 101.27) (width 0.4) (layer "B.Cu") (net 6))
 (segment (start 151.22 100.21) (end 156.44 100.21) (width 0.4) (layer "B.Cu") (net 6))
 (segment (start 132.32 102.52) (end 135.64 99.2) (width 0.4) (layer "B.Cu") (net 5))
 (segment (start 159.39 101.8) (end 159.6 101.8) (width 0.4) (layer "B.Cu") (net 5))
 (segment (start 135.64 99.2) (end 156.79 99.2) (width 0.4) (layer "B.Cu") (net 5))
 (segment (start 156.79 99.2) (end 159.39 101.8) (width 0.4) (layer "B.Cu") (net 5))
 (segment (start 132.32 108.08) (end 132.32 102.52) (width 0.4) (layer "B.Cu") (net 5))
 (segment (start 160.3875 82.4625) (end 159.1 83.75) (width 0.4) (layer "F.Cu") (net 3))
 (segment (start 159.1 83.75) (end 159.1 90.25) (width 0.4) (layer "F.Cu") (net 3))
 (segment (start 160.3875 81.55) (end 160.3875 82.4625) (width 0.4) (layer "F.Cu") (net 3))
 (segment (start 154.74 86.55) (end 157.54 83.75) (width 0.4) (layer "B.Cu") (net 3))
 (segment (start 152.95 86.55) (end 154.74 86.55) (width 0.4) (layer "B.Cu") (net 3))
 (segment (start 148.63 82.23) (end 152.95 86.55) (width 0.4) (layer "B.Cu") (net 3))
 (segment (start 157.54 83.75) (end 159.1 83.75) (width 0.4) (layer "B.Cu") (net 3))
 (segment (start 166.76 84.27) (end 166.76 86.115) (width 0.4) (layer "F.Cu") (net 9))
 (via (at 166.76 84.27) (size 0.7) (drill 0.3) (layers "F.Cu" "B.Cu") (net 9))
 (segment (start 158.99 88.63) (end 139.3 88.63) (width 0.4) (layer "B.Cu") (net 9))
 (segment (start 139.3 88.63) (end 137.26 86.59) (width 0.4) (layer "B.Cu") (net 9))
 (segment (start 166.76 84.27) (end 165.14 85.89) (width 0.4) (layer "B.Cu") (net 9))
 (segment (start 137.26 86.59) (end 137.26 83.44) (width 0.4) (layer "B.Cu") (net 9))
 (segment (start 165.14 85.89) (end 161.73 85.89) (width 0.4) (layer "B.Cu") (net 9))
 (segment (start 137.26 83.44) (end 138.47 82.23) (width 0.4) (layer "B.Cu") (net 9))
 (segment (start 161.73 85.89) (end 158.99 88.63) (width 0.4) (layer "B.Cu") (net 9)))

